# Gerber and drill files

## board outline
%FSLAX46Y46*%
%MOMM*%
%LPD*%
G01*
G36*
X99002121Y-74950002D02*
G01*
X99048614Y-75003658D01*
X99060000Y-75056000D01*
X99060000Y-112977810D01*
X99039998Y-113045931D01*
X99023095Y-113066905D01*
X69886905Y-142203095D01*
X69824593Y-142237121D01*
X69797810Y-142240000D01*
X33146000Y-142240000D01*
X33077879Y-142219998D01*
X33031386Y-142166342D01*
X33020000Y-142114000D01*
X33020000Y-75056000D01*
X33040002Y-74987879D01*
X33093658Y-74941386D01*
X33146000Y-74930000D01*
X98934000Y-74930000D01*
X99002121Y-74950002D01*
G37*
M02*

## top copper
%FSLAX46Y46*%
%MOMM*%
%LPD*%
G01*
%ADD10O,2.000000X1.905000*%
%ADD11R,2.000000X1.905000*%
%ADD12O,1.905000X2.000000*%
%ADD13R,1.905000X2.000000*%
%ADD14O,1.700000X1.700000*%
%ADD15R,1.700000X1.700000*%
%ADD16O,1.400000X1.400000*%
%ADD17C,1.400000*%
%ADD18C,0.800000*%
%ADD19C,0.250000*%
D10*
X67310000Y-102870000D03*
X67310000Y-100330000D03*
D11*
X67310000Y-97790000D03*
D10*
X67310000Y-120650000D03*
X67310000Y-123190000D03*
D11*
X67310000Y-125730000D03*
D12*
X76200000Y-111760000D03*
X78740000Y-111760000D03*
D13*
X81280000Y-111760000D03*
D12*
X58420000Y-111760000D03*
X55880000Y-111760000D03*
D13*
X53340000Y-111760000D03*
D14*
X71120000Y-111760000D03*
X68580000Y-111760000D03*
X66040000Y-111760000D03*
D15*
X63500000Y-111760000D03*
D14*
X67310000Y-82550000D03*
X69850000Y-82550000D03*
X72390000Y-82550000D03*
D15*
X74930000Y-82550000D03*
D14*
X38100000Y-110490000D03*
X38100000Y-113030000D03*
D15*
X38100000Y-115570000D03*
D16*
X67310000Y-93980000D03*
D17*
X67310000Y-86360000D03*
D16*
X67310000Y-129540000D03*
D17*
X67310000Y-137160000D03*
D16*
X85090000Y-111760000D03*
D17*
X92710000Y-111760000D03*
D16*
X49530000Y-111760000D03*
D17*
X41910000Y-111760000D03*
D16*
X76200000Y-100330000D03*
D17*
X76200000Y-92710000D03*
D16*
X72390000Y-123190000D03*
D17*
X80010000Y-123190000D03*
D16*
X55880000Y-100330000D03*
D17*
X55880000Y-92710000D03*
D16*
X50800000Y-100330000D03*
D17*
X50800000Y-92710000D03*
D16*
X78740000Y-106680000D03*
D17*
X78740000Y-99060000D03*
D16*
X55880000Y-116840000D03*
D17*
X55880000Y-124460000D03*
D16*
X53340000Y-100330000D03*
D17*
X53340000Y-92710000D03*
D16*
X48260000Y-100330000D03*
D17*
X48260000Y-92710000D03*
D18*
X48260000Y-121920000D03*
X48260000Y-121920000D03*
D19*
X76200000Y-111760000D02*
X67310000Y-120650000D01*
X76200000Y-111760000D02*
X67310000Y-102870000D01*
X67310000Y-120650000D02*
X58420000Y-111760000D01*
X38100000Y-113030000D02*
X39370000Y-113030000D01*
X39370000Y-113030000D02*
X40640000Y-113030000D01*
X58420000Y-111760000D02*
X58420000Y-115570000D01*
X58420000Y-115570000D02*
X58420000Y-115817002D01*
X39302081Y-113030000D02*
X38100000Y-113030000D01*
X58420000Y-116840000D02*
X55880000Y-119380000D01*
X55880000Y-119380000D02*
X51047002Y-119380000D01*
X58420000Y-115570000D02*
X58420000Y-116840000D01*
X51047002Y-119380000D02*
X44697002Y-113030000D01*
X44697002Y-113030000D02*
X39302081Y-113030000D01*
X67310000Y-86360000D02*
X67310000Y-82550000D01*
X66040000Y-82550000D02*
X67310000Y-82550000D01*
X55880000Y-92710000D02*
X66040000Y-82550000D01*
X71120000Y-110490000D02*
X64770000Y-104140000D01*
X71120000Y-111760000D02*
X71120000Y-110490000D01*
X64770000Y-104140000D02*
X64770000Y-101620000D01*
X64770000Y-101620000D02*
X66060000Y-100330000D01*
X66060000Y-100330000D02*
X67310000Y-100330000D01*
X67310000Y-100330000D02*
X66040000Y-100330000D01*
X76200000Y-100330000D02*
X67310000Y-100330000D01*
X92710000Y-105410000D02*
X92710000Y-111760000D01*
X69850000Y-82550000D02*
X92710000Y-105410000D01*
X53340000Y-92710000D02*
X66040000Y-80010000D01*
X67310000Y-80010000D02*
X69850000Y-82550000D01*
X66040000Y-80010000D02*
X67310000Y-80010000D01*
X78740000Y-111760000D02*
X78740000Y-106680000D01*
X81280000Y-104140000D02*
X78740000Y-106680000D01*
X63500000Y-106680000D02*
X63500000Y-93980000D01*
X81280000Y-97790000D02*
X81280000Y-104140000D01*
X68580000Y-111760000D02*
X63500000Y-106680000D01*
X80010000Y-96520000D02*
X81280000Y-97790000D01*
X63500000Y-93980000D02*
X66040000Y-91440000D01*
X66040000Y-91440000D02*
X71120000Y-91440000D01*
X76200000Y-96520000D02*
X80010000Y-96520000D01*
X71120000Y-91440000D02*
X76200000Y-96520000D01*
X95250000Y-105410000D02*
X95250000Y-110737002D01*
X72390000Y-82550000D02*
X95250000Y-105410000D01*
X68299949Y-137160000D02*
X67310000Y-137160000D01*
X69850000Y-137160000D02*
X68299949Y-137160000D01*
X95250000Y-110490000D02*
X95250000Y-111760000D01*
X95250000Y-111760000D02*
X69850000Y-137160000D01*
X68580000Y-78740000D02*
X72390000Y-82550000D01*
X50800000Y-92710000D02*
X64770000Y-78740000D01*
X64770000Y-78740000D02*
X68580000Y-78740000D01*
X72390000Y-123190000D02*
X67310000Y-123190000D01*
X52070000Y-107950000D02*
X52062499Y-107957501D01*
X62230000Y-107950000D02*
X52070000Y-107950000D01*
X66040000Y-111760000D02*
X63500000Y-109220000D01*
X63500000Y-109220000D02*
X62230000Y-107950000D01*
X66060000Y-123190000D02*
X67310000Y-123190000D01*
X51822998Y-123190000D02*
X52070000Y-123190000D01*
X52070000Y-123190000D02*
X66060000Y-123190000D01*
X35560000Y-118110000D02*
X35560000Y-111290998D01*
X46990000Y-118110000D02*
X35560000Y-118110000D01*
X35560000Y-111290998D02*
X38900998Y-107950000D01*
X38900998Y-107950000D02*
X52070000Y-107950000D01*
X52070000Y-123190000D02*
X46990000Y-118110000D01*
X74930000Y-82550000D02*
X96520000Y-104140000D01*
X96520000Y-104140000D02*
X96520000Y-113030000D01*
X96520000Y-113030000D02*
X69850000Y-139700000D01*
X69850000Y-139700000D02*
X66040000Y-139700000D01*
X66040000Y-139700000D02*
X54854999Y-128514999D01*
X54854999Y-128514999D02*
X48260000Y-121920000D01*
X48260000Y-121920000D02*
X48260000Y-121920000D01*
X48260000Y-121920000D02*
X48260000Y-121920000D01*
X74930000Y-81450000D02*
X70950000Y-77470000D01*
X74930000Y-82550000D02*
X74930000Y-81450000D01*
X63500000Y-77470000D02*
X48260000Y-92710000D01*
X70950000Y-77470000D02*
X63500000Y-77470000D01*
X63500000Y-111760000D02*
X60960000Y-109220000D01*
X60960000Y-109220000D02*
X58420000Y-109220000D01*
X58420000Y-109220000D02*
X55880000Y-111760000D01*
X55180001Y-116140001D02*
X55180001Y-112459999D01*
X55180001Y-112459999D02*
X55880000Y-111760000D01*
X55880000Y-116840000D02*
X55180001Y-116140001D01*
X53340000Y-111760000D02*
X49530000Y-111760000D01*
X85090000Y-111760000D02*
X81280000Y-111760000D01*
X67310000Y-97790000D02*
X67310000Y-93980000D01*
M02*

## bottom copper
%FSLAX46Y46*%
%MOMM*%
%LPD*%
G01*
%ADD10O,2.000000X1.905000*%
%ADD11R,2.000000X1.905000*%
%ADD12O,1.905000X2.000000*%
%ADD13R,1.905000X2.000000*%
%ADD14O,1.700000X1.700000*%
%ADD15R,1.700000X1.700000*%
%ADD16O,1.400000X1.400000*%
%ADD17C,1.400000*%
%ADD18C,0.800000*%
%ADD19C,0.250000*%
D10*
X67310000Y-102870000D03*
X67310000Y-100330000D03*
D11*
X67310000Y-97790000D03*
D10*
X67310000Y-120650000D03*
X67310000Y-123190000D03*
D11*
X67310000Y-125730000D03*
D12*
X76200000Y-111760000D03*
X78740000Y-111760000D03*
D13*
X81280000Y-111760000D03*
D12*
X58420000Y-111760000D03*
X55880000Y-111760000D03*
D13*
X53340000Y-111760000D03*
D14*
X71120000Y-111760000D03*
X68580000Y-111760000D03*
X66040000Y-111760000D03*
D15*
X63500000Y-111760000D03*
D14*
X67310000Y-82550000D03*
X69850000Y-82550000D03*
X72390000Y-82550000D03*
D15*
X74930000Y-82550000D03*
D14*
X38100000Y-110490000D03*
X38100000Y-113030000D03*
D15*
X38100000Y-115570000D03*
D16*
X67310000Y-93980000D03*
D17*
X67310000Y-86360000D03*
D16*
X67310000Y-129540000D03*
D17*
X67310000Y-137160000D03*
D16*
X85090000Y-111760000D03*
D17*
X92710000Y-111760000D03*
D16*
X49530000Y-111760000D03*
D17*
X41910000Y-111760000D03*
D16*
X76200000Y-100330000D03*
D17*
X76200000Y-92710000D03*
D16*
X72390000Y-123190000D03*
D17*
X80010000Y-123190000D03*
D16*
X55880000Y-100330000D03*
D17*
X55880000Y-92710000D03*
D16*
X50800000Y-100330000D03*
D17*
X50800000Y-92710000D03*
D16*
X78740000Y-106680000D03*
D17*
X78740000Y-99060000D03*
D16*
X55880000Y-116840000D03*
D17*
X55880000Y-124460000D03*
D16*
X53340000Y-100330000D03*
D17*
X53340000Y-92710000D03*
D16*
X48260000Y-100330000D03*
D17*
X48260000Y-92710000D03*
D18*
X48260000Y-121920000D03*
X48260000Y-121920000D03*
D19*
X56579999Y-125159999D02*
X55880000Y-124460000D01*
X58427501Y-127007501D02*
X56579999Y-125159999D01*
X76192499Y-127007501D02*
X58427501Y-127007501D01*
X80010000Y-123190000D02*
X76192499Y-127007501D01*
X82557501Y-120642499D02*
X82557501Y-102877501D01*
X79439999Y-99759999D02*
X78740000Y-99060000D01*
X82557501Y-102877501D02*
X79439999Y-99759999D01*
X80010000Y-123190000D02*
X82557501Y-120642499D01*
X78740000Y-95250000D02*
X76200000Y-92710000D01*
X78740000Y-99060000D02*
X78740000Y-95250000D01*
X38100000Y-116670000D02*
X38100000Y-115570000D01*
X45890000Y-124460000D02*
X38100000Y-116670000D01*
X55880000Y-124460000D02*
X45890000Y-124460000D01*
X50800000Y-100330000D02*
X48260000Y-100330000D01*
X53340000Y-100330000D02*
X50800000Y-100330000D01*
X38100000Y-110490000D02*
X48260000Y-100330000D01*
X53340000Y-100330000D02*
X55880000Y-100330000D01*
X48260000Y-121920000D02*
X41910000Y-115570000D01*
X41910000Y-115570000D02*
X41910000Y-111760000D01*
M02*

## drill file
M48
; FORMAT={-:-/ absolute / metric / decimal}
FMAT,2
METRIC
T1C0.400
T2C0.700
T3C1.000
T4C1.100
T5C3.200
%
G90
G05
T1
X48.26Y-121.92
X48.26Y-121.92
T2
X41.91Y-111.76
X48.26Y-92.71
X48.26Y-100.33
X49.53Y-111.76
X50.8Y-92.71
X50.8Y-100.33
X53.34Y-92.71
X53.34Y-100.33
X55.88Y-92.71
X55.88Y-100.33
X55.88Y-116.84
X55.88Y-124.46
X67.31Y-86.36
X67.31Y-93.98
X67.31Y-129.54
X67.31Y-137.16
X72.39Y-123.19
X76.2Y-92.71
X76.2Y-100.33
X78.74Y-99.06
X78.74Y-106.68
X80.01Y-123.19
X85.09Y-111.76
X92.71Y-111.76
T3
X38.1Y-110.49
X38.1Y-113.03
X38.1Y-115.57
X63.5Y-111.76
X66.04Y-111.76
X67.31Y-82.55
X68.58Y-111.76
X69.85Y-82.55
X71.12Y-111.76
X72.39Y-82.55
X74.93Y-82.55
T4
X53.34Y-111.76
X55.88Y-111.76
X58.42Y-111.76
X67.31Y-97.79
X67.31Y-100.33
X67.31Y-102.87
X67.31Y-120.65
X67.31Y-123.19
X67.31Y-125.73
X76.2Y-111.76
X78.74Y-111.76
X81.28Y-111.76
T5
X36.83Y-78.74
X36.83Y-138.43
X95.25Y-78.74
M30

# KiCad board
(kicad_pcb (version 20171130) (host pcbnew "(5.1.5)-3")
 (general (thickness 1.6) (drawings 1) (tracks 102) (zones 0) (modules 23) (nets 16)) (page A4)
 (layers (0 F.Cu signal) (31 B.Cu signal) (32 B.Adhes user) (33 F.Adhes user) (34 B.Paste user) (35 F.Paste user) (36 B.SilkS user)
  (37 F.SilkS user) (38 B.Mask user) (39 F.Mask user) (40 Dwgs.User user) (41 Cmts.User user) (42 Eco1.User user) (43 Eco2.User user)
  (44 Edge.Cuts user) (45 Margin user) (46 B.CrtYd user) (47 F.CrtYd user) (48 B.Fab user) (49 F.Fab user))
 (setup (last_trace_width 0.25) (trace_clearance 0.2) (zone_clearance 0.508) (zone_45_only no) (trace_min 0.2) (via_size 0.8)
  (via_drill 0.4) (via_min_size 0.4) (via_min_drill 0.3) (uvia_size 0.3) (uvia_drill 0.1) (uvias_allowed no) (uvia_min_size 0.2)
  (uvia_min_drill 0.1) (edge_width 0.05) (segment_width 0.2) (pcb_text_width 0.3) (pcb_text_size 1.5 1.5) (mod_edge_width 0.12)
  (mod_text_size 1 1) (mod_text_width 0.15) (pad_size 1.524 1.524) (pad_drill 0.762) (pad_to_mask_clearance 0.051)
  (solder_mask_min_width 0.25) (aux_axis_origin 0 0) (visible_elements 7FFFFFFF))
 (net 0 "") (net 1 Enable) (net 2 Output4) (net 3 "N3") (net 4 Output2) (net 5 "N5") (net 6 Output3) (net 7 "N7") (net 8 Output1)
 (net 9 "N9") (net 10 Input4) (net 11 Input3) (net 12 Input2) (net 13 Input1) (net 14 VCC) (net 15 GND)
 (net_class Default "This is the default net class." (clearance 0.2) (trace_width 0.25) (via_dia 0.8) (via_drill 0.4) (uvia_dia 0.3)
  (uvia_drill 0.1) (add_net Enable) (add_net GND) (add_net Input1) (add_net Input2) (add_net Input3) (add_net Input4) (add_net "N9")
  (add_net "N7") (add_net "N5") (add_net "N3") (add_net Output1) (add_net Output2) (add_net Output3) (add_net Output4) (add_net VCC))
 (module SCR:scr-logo (layer F.Cu) (at 46.99 82.55)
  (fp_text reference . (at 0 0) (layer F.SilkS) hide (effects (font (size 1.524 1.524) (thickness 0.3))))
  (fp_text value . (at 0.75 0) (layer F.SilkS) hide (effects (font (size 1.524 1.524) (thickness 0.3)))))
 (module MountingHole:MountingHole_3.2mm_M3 (layer F.Cu) (at 95.25 78.74)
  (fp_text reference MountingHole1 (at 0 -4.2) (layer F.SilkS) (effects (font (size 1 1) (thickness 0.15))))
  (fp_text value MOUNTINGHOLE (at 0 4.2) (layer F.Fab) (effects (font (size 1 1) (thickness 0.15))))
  (pad 1 np_thru_hole circle (at 0 0) (size 3.2 3.2) (drill 3.2) (layers *.Cu *.Mask)))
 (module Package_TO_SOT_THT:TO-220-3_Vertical (layer B.Cu) (at 67.31 97.79 270)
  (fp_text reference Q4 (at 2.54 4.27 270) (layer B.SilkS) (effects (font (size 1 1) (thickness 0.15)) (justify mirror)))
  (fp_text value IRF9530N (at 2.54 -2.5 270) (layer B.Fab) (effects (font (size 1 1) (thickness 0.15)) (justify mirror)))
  (pad 3 thru_hole oval (at 5.08 0 270) (size 1.905 2) (drill 1.1) (layers *.Cu *.Mask) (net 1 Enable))
  (pad 2 thru_hole oval (at 2.54 0 270) (size 1.905 2) (drill 1.1) (layers *.Cu *.Mask) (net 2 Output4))
  (pad 1 thru_hole rect (at 0 0 270) (size 1.905 2) (drill 1.1) (layers *.Cu *.Mask) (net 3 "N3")))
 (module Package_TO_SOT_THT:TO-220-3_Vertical (layer B.Cu) (at 67.31 125.73 90)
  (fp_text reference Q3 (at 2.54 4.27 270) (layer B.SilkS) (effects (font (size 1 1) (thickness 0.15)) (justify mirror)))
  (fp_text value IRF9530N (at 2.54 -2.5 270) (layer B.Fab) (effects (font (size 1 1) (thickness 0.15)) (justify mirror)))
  (pad 3 thru_hole oval (at 5.08 0 90) (size 1.905 2) (drill 1.1) (layers *.Cu *.Mask) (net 1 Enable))
  (pad 2 thru_hole oval (at 2.54 0 90) (size 1.905 2) (drill 1.1) (layers *.Cu *.Mask) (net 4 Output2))
  (pad 1 thru_hole rect (at 0 0 90) (size 1.905 2) (drill 1.1) (layers *.Cu *.Mask) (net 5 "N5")))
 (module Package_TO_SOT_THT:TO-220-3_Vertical (layer B.Cu) (at 81.28 111.76 180)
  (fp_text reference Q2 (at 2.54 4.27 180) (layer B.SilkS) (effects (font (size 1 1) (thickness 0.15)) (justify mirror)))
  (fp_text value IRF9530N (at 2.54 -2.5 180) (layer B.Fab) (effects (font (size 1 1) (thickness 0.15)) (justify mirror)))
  (pad 3 thru_hole oval (at 5.08 0 180) (size 1.905 2) (drill 1.1) (layers *.Cu *.Mask) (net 1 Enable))
  (pad 2 thru_hole oval (at 2.54 0 180) (size 1.905 2) (drill 1.1) (layers *.Cu *.Mask) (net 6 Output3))
  (pad 1 thru_hole rect (at 0 0 180) (size 1.905 2) (drill 1.1) (layers *.Cu *.Mask) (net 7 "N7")))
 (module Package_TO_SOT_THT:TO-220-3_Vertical (layer B.Cu) (at 53.34 111.76)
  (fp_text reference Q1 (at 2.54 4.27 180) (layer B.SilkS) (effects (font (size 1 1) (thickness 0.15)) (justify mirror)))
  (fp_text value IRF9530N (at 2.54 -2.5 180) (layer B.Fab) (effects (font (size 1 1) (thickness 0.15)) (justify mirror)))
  (pad 3 thru_hole oval (at 5.08 0) (size 1.905 2) (drill 1.1) (layers *.Cu *.Mask) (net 1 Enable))
  (pad 2 thru_hole oval (at 2.54 0) (size 1.905 2) (drill 1.1) (layers *.Cu *.Mask) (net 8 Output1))
  (pad 1 thru_hole rect (at 0 0) (size 1.905 2) (drill 1.1) (layers *.Cu *.Mask) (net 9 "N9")))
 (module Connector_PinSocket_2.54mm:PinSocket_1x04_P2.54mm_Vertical (layer F.Cu) (at 63.5 111.76 90)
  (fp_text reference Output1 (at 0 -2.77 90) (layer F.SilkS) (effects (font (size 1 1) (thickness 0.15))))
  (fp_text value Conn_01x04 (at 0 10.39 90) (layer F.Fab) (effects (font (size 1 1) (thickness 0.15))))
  (pad 4 thru_hole oval (at 0 7.62 90) (size 1.7 1.7) (drill 1) (layers *.Cu *.Mask) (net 2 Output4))
  (pad 3 thru_hole oval (at 0 5.08 90) (size 1.7 1.7) (drill 1) (layers *.Cu *.Mask) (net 6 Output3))
  (pad 2 thru_hole oval (at 0 2.54 90) (size 1.7 1.7) (drill 1) (layers *.Cu *.Mask) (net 4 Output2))
  (pad 1 thru_hole rect (at 0 0 90) (size 1.7 1.7) (drill 1) (layers *.Cu *.Mask) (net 8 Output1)))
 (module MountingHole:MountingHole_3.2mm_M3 (layer F.Cu) (at 36.83 138.43)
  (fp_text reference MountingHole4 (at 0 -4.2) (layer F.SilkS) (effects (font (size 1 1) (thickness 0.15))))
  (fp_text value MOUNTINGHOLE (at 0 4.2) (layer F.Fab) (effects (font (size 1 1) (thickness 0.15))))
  (pad 1 np_thru_hole circle (at 0 0) (size 3.2 3.2) (drill 3.2) (layers *.Cu *.Mask)))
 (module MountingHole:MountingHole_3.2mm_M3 (layer F.Cu) (at 36.83 78.74)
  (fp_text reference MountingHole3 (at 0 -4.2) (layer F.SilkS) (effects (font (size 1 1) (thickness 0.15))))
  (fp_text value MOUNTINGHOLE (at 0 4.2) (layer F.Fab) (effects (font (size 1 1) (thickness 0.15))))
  (pad 1 np_thru_hole circle (at 0 0) (size 3.2 3.2) (drill 3.2) (layers *.Cu *.Mask)))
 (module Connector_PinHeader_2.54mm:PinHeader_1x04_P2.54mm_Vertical (layer F.Cu) (at 74.93 82.55 270)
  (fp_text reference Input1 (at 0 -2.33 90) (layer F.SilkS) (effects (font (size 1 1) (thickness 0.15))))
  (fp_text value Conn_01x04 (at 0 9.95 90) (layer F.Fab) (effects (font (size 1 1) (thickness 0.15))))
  (pad 4 thru_hole oval (at 0 7.62 270) (size 1.7 1.7) (drill 1) (layers *.Cu *.Mask) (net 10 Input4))
  (pad 3 thru_hole oval (at 0 5.08 270) (size 1.7 1.7) (drill 1) (layers *.Cu *.Mask) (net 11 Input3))
  (pad 2 thru_hole oval (at 0 2.54 270) (size 1.7 1.7) (drill 1) (layers *.Cu *.Mask) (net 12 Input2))
  (pad 1 thru_hole rect (at 0 0 270) (size 1.7 1.7) (drill 1) (layers *.Cu *.Mask) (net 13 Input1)))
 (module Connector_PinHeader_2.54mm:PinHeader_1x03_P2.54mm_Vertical (layer F.Cu) (at 38.1 115.57 180)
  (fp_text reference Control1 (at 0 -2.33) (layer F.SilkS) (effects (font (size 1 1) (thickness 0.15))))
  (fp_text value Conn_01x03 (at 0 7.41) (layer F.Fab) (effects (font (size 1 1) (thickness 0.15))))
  (pad 3 thru_hole oval (at 0 5.08 180) (size 1.7 1.7) (drill 1) (layers *.Cu *.Mask) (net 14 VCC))
  (pad 2 thru_hole oval (at 0 2.54 180) (size 1.7 1.7) (drill 1) (layers *.Cu *.Mask) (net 1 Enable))
  (pad 1 thru_hole rect (at 0 0 180) (size 1.7 1.7) (drill 1) (layers *.Cu *.Mask) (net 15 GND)))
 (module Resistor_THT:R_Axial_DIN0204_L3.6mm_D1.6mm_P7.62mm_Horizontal (layer F.Cu) (at 67.31 86.36 270)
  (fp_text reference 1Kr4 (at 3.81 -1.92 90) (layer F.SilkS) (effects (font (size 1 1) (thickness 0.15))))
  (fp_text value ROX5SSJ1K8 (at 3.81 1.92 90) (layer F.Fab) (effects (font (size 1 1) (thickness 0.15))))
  (pad 2 thru_hole oval (at 7.62 0 270) (size 1.4 1.4) (drill 0.7) (layers *.Cu *.Mask) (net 3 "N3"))
  (pad 1 thru_hole circle (at 0 0 270) (size 1.4 1.4) (drill 0.7) (layers *.Cu *.Mask) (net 10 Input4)))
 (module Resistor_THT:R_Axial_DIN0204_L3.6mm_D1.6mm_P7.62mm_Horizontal (layer F.Cu) (at 67.31 137.16 90)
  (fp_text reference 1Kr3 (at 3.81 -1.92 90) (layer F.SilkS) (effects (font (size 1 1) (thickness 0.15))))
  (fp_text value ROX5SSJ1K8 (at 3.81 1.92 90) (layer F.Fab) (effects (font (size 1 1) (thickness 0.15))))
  (pad 2 thru_hole oval (at 7.62 0 90) (size 1.4 1.4) (drill 0.7) (layers *.Cu *.Mask) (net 5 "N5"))
  (pad 1 thru_hole circle (at 0 0 90) (size 1.4 1.4) (drill 0.7) (layers *.Cu *.Mask) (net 12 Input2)))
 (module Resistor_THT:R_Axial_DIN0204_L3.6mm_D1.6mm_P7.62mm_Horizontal (layer F.Cu) (at 92.71 111.76 180)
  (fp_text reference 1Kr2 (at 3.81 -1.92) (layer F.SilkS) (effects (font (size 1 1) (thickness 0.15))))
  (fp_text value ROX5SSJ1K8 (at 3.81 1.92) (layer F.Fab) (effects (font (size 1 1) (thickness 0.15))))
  (pad 2 thru_hole oval (at 7.62 0 180) (size 1.4 1.4) (drill 0.7) (layers *.Cu *.Mask) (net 7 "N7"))
  (pad 1 thru_hole circle (at 0 0 180) (size 1.4 1.4) (drill 0.7) (layers *.Cu *.Mask) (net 11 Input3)))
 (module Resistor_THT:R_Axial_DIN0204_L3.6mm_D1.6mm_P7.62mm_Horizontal (layer F.Cu) (at 41.91 111.76)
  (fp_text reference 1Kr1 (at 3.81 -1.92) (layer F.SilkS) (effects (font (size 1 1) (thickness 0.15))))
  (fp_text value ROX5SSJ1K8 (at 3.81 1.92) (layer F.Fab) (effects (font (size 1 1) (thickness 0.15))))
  (pad 2 thru_hole oval (at 7.62 0) (size 1.4 1.4) (drill 0.7) (layers *.Cu *.Mask) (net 9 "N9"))
  (pad 1 thru_hole circle (at 0 0) (size 1.4 1.4) (drill 0.7) (layers *.Cu *.Mask) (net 13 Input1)))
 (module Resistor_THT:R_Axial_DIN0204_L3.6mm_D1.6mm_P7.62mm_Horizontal (layer F.Cu) (at 76.2 92.71 270)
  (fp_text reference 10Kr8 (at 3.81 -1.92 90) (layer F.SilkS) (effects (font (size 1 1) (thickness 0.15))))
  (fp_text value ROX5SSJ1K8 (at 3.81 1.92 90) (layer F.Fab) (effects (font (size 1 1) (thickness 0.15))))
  (pad 2 thru_hole oval (at 7.62 0 270) (size 1.4 1.4) (drill 0.7) (layers *.Cu *.Mask) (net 2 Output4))
  (pad 1 thru_hole circle (at 0 0 270) (size 1.4 1.4) (drill 0.7) (layers *.Cu *.Mask) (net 15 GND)))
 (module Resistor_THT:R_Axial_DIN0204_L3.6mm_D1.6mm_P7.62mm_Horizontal (layer F.Cu) (at 80.01 123.19 180)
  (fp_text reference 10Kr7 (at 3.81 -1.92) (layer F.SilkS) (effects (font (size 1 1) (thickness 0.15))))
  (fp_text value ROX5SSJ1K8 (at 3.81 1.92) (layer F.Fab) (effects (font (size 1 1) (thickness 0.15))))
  (pad 2 thru_hole oval (at 7.62 0 180) (size 1.4 1.4) (drill 0.7) (layers *.Cu *.Mask) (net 4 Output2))
  (pad 1 thru_hole circle (at 0 0 180) (size 1.4 1.4) (drill 0.7) (layers *.Cu *.Mask) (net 15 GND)))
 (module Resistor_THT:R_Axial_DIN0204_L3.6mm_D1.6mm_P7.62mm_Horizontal (layer F.Cu) (at 55.88 92.71 270)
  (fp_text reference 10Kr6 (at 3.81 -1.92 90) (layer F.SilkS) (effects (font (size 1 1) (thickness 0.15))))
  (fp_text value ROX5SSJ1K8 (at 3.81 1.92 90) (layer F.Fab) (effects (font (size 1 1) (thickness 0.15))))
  (pad 2 thru_hole oval (at 7.62 0 270) (size 1.4 1.4) (drill 0.7) (layers *.Cu *.Mask) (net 14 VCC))
  (pad 1 thru_hole circle (at 0 0 270) (size 1.4 1.4) (drill 0.7) (layers *.Cu *.Mask) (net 10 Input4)))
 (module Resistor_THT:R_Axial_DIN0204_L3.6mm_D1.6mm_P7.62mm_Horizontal (layer F.Cu) (at 50.8 92.71 270)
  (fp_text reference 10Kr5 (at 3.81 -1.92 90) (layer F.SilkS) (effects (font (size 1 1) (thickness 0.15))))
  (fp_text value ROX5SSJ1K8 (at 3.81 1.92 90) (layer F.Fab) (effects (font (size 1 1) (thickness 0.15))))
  (pad 2 thru_hole oval (at 7.62 0 270) (size 1.4 1.4) (drill 0.7) (layers *.Cu *.Mask) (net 14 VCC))
  (pad 1 thru_hole circle (at 0 0 270) (size 1.4 1.4) (drill 0.7) (layers *.Cu *.Mask) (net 12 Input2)))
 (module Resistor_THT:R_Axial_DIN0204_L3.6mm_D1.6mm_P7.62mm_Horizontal (layer F.Cu) (at 78.74 99.06 270)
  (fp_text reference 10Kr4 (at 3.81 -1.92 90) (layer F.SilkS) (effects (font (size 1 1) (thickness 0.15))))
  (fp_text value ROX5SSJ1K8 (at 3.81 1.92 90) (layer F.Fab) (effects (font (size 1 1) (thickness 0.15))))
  (pad 2 thru_hole oval (at 7.62 0 270) (size 1.4 1.4) (drill 0.7) (layers *.Cu *.Mask) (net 6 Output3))
  (pad 1 thru_hole circle (at 0 0 270) (size 1.4 1.4) (drill 0.7) (layers *.Cu *.Mask) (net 15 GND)))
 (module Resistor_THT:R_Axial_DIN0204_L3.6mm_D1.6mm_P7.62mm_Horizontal (layer F.Cu) (at 55.88 124.46 90)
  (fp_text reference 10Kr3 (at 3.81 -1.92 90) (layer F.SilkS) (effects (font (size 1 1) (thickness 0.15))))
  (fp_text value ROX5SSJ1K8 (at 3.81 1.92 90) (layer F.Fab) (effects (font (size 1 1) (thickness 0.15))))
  (pad 2 thru_hole oval (at 7.62 0 90) (size 1.4 1.4) (drill 0.7) (layers *.Cu *.Mask) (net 8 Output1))
  (pad 1 thru_hole circle (at 0 0 90) (size 1.4 1.4) (drill 0.7) (layers *.Cu *.Mask) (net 15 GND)))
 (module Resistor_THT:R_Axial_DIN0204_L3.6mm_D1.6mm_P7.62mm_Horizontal (layer F.Cu) (at 53.34 92.71 270)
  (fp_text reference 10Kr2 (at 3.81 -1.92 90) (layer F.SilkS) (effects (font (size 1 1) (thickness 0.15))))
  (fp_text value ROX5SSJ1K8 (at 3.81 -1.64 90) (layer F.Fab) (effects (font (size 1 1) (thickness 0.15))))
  (pad 2 thru_hole oval (at 7.62 0 270) (size 1.4 1.4) (drill 0.7) (layers *.Cu *.Mask) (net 14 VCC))
  (pad 1 thru_hole circle (at 0 0 270) (size 1.4 1.4) (drill 0.7) (layers *.Cu *.Mask) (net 11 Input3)))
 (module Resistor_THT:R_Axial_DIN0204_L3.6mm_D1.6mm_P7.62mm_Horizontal (layer F.Cu) (at 48.26 92.71 270)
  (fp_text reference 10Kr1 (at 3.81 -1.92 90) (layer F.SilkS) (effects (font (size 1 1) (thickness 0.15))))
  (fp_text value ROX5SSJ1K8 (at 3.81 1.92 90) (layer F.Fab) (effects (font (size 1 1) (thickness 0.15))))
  (pad 2 thru_hole oval (at 7.62 0 270) (size 1.4 1.4) (drill 0.7) (layers *.Cu *.Mask) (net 14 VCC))
  (pad 1 thru_hole circle (at 0 0 270) (size 1.4 1.4) (drill 0.7) (layers *.Cu *.Mask) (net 13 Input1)))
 (segment (start 76.2 111.76) (end 67.31 120.65) (width 0.25) (layer F.Cu) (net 1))
 (segment (start 76.2 111.76) (end 67.31 102.87) (width 0.25) (layer F.Cu) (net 1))
 (segment (start 67.31 120.65) (end 58.42 111.76) (width 0.25) (layer F.Cu) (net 1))
 (segment (start 38.1 113.03) (end 39.37 113.03) (width 0.25) (layer F.Cu) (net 1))
 (segment (start 39.37 113.03) (end 40.64 113.03) (width 0.25) (layer F.Cu) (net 1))
 (segment (start 58.42 111.76) (end 58.42 115.57) (width 0.25) (layer F.Cu) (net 1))
 (segment (start 58.42 115.57) (end 58.42 115.817002) (width 0.25) (layer F.Cu) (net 1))
 (segment (start 39.302081 113.03) (end 38.1 113.03) (width 0.25) (layer F.Cu) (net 1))
 (segment (start 58.42 116.84) (end 55.88 119.38) (width 0.25) (layer F.Cu) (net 1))
 (segment (start 55.88 119.38) (end 51.047002 119.38) (width 0.25) (layer F.Cu) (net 1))
 (segment (start 58.42 115.57) (end 58.42 116.84) (width 0.25) (layer F.Cu) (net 1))
 (segment (start 51.047002 119.38) (end 44.697002 113.03) (width 0.25) (layer F.Cu) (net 1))
 (segment (start 44.697002 113.03) (end 39.302081 113.03) (width 0.25) (layer F.Cu) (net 1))
 (segment (start 56.579999 125.159999) (end 55.88 124.46) (width 0.25) (layer B.Cu) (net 15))
 (segment (start 58.427501 127.007501) (end 56.579999 125.159999) (width 0.25) (layer B.Cu) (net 15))
 (segment (start 76.192499 127.007501) (end 58.427501 127.007501) (width 0.25) (layer B.Cu) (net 15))
 (segment (start 80.01 123.19) (end 76.192499 127.007501) (width 0.25) (layer B.Cu) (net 15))
 (segment (start 82.557501 120.642499) (end 82.557501 102.877501) (width 0.25) (layer B.Cu) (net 15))
 (segment (start 79.439999 99.759999) (end 78.74 99.06) (width 0.25) (layer B.Cu) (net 15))
 (segment (start 82.557501 102.877501) (end 79.439999 99.759999) (width 0.25) (layer B.Cu) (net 15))
 (segment (start 80.01 123.19) (end 82.557501 120.642499) (width 0.25) (layer B.Cu) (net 15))
 (segment (start 78.74 95.25) (end 76.2 92.71) (width 0.25) (layer B.Cu) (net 15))
 (segment (start 78.74 99.06) (end 78.74 95.25) (width 0.25) (layer B.Cu) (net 15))
 (segment (start 38.1 116.67) (end 38.1 115.57) (width 0.25) (layer B.Cu) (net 15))
 (segment (start 45.89 124.46) (end 38.1 116.67) (width 0.25) (layer B.Cu) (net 15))
 (segment (start 55.88 124.46) (end 45.89 124.46) (width 0.25) (layer B.Cu) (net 15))
 (segment (start 50.8 100.33) (end 48.26 100.33) (width 0.25) (layer B.Cu) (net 14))
 (segment (start 53.34 100.33) (end 50.8 100.33) (width 0.25) (layer B.Cu) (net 14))
 (segment (start 38.1 110.49) (end 48.26 100.33) (width 0.25) (layer B.Cu) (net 14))
 (segment (start 53.34 100.33) (end 55.88 100.33) (width 0.25) (layer B.Cu) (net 14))
 (segment (start 67.31 86.36) (end 67.31 82.55) (width 0.25) (layer F.Cu) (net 10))
 (segment (start 66.04 82.55) (end 67.31 82.55) (width 0.25) (layer F.Cu) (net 10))
 (segment (start 55.88 92.71) (end 66.04 82.55) (width 0.25) (layer F.Cu) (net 10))
 (segment (start 71.12 110.49) (end 64.77 104.14) (width 0.25) (layer F.Cu) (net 2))
 (segment (start 71.12 111.76) (end 71.12 110.49) (width 0.25) (layer F.Cu) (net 2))
 (segment (start 64.77 104.14) (end 64.77 101.62) (width 0.25) (layer F.Cu) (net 2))
 (segment (start 64.77 101.62) (end 66.06 100.33) (width 0.25) (layer F.Cu) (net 2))
 (segment (start 66.06 100.33) (end 67.31 100.33) (width 0.25) (layer F.Cu) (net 2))
 (segment (start 67.31 100.33) (end 66.04 100.33) (width 0.25) (layer F.Cu) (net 2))
 (segment (start 76.2 100.33) (end 67.31 100.33) (width 0.25) (layer F.Cu) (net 2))
 (segment (start 92.71 105.41) (end 92.71 111.76) (width 0.25) (layer F.Cu) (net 11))
 (segment (start 69.85 82.55) (end 92.71 105.41) (width 0.25) (layer F.Cu) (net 11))
 (segment (start 53.34 92.71) (end 66.04 80.01) (width 0.25) (layer F.Cu) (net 11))
 (segment (start 67.31 80.01) (end 69.85 82.55) (width 0.25) (layer F.Cu) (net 11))
 (segment (start 66.04 80.01) (end 67.31 80.01) (width 0.25) (layer F.Cu) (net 11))
 (segment (start 78.74 111.76) (end 78.74 106.68) (width 0.25) (layer F.Cu) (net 6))
 (segment (start 81.28 104.14) (end 78.74 106.68) (width 0.25) (layer F.Cu) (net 6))
 (segment (start 63.5 106.68) (end 63.5 93.98) (width 0.25) (layer F.Cu) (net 6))
 (segment (start 81.28 97.79) (end 81.28 104.14) (width 0.25) (layer F.Cu) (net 6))
 (segment (start 68.58 111.76) (end 63.5 106.68) (width 0.25) (layer F.Cu) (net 6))
 (segment (start 80.01 96.52) (end 81.28 97.79) (width 0.25) (layer F.Cu) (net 6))
 (segment (start 63.5 93.98) (end 66.04 91.44) (width 0.25) (layer F.Cu) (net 6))
 (segment (start 66.04 91.44) (end 71.12 91.44) (width 0.25) (layer F.Cu) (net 6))
 (segment (start 76.2 96.52) (end 80.01 96.52) (width 0.25) (layer F.Cu) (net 6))
 (segment (start 71.12 91.44) (end 76.2 96.52) (width 0.25) (layer F.Cu) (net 6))
 (segment (start 95.25 105.41) (end 95.25 110.737002) (width 0.25) (layer F.Cu) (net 12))
 (segment (start 72.39 82.55) (end 95.25 105.41) (width 0.25) (layer F.Cu) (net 12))
 (segment (start 68.299949 137.16) (end 67.31 137.16) (width 0.25) (layer F.Cu) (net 12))
 (segment (start 69.85 137.16) (end 68.299949 137.16) (width 0.25) (layer F.Cu) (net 12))
 (segment (start 95.25 110.49) (end 95.25 111.76) (width 0.25) (layer F.Cu) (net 12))
 (segment (start 95.25 111.76) (end 69.85 137.16) (width 0.25) (layer F.Cu) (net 12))
 (segment (start 68.58 78.74) (end 72.39 82.55) (width 0.25) (layer F.Cu) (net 12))
 (segment (start 50.8 92.71) (end 64.77 78.74) (width 0.25) (layer F.Cu) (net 12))
 (segment (start 64.77 78.74) (end 68.58 78.74) (width 0.25) (layer F.Cu) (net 12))
 (segment (start 72.39 123.19) (end 67.31 123.19) (width 0.25) (layer F.Cu) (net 4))
 (segment (start 52.07 107.95) (end 52.062499 107.957501) (width 0.25) (layer F.Cu) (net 4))
 (segment (start 62.23 107.95) (end 52.07 107.95) (width 0.25) (layer F.Cu) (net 4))
 (segment (start 66.04 111.76) (end 63.5 109.22) (width 0.25) (layer F.Cu) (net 4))
 (segment (start 63.5 109.22) (end 62.23 107.95) (width 0.25) (layer F.Cu) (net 4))
 (segment (start 66.06 123.19) (end 67.31 123.19) (width 0.25) (layer F.Cu) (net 4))
 (segment (start 51.822998 123.19) (end 52.07 123.19) (width 0.25) (layer F.Cu) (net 4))
 (segment (start 52.07 123.19) (end 66.06 123.19) (width 0.25) (layer F.Cu) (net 4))
 (segment (start 35.56 118.11) (end 35.56 111.290998) (width 0.25) (layer F.Cu) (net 4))
 (segment (start 46.99 118.11) (end 35.56 118.11) (width 0.25) (layer F.Cu) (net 4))
 (segment (start 35.56 111.290998) (end 38.900998 107.95) (width 0.25) (layer F.Cu) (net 4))
 (segment (start 38.900998 107.95) (end 52.07 107.95) (width 0.25) (layer F.Cu) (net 4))
 (segment (start 52.07 123.19) (end 46.99 118.11) (width 0.25) (layer F.Cu) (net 4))
 (segment (start 74.93 82.55) (end 96.52 104.14) (width 0.25) (layer F.Cu) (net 13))
 (segment (start 96.52 104.14) (end 96.52 113.03) (width 0.25) (layer F.Cu) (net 13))
 (segment (start 96.52 113.03) (end 69.85 139.7) (width 0.25) (layer F.Cu) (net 13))
 (segment (start 69.85 139.7) (end 66.04 139.7) (width 0.25) (layer F.Cu) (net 13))
 (segment (start 66.04 139.7) (end 54.854999 128.514999) (width 0.25) (layer F.Cu) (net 13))
 (segment (start 54.854999 128.514999) (end 48.26 121.92) (width 0.25) (layer F.Cu) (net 13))
 (segment (start 48.26 121.92) (end 48.26 121.92) (width 0.25) (layer F.Cu) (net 13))
 (via (at 48.26 121.92) (size 0.8) (drill 0.4) (layers F.Cu B.Cu) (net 13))
 (segment (start 48.26 121.92) (end 48.26 121.92) (width 0.25) (layer F.Cu) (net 13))
 (via (at 48.26 121.92) (size 0.8) (drill 0.4) (layers F.Cu B.Cu) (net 13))
 (segment (start 48.26 121.92) (end 41.91 115.57) (width 0.25) (layer B.Cu) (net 13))
 (segment (start 41.91 115.57) (end 41.91 111.76) (width 0.25) (layer B.Cu) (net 13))
 (segment (start 74.93 81.45) (end 70.95 77.47) (width 0.25) (layer F.Cu) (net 13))
 (segment (start 74.93 82.55) (end 74.93 81.45) (width 0.25) (layer F.Cu) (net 13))
 (segment (start 63.5 77.47) (end 48.26 92.71) (width 0.25) (layer F.Cu) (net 13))
 (segment (start 70.95 77.47) (end 63.5 77.47) (width 0.25) (layer F.Cu) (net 13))
 (segment (start 63.5 111.76) (end 60.96 109.22) (width 0.25) (layer F.Cu) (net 8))
 (segment (start 60.96 109.22) (end 58.42 109.22) (width 0.25) (layer F.Cu) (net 8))
 (segment (start 58.42 109.22) (end 55.88 111.76) (width 0.25) (layer F.Cu) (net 8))
 (segment (start 55.180001 116.140001) (end 55.180001 112.459999) (width 0.25) (layer F.Cu) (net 8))
 (segment (start 55.180001 112.459999) (end 55.88 111.76) (width 0.25) (layer F.Cu) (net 8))
 (segment (start 55.88 116.84) (end 55.180001 116.140001) (width 0.25) (layer F.Cu) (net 8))
 (segment (start 53.34 111.76) (end 49.53 111.76) (width 0.25) (layer F.Cu) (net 9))
 (segment (start 85.09 111.76) (end 81.28 111.76) (width 0.25) (layer F.Cu) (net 7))
 (segment (start 67.31 97.79) (end 67.31 93.98) (width 0.25) (layer F.Cu) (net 3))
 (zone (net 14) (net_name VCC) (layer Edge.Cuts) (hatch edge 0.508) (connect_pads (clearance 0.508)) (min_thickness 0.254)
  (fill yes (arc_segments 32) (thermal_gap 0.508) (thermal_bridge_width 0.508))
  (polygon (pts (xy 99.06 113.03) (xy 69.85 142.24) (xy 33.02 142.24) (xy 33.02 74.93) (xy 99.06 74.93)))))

